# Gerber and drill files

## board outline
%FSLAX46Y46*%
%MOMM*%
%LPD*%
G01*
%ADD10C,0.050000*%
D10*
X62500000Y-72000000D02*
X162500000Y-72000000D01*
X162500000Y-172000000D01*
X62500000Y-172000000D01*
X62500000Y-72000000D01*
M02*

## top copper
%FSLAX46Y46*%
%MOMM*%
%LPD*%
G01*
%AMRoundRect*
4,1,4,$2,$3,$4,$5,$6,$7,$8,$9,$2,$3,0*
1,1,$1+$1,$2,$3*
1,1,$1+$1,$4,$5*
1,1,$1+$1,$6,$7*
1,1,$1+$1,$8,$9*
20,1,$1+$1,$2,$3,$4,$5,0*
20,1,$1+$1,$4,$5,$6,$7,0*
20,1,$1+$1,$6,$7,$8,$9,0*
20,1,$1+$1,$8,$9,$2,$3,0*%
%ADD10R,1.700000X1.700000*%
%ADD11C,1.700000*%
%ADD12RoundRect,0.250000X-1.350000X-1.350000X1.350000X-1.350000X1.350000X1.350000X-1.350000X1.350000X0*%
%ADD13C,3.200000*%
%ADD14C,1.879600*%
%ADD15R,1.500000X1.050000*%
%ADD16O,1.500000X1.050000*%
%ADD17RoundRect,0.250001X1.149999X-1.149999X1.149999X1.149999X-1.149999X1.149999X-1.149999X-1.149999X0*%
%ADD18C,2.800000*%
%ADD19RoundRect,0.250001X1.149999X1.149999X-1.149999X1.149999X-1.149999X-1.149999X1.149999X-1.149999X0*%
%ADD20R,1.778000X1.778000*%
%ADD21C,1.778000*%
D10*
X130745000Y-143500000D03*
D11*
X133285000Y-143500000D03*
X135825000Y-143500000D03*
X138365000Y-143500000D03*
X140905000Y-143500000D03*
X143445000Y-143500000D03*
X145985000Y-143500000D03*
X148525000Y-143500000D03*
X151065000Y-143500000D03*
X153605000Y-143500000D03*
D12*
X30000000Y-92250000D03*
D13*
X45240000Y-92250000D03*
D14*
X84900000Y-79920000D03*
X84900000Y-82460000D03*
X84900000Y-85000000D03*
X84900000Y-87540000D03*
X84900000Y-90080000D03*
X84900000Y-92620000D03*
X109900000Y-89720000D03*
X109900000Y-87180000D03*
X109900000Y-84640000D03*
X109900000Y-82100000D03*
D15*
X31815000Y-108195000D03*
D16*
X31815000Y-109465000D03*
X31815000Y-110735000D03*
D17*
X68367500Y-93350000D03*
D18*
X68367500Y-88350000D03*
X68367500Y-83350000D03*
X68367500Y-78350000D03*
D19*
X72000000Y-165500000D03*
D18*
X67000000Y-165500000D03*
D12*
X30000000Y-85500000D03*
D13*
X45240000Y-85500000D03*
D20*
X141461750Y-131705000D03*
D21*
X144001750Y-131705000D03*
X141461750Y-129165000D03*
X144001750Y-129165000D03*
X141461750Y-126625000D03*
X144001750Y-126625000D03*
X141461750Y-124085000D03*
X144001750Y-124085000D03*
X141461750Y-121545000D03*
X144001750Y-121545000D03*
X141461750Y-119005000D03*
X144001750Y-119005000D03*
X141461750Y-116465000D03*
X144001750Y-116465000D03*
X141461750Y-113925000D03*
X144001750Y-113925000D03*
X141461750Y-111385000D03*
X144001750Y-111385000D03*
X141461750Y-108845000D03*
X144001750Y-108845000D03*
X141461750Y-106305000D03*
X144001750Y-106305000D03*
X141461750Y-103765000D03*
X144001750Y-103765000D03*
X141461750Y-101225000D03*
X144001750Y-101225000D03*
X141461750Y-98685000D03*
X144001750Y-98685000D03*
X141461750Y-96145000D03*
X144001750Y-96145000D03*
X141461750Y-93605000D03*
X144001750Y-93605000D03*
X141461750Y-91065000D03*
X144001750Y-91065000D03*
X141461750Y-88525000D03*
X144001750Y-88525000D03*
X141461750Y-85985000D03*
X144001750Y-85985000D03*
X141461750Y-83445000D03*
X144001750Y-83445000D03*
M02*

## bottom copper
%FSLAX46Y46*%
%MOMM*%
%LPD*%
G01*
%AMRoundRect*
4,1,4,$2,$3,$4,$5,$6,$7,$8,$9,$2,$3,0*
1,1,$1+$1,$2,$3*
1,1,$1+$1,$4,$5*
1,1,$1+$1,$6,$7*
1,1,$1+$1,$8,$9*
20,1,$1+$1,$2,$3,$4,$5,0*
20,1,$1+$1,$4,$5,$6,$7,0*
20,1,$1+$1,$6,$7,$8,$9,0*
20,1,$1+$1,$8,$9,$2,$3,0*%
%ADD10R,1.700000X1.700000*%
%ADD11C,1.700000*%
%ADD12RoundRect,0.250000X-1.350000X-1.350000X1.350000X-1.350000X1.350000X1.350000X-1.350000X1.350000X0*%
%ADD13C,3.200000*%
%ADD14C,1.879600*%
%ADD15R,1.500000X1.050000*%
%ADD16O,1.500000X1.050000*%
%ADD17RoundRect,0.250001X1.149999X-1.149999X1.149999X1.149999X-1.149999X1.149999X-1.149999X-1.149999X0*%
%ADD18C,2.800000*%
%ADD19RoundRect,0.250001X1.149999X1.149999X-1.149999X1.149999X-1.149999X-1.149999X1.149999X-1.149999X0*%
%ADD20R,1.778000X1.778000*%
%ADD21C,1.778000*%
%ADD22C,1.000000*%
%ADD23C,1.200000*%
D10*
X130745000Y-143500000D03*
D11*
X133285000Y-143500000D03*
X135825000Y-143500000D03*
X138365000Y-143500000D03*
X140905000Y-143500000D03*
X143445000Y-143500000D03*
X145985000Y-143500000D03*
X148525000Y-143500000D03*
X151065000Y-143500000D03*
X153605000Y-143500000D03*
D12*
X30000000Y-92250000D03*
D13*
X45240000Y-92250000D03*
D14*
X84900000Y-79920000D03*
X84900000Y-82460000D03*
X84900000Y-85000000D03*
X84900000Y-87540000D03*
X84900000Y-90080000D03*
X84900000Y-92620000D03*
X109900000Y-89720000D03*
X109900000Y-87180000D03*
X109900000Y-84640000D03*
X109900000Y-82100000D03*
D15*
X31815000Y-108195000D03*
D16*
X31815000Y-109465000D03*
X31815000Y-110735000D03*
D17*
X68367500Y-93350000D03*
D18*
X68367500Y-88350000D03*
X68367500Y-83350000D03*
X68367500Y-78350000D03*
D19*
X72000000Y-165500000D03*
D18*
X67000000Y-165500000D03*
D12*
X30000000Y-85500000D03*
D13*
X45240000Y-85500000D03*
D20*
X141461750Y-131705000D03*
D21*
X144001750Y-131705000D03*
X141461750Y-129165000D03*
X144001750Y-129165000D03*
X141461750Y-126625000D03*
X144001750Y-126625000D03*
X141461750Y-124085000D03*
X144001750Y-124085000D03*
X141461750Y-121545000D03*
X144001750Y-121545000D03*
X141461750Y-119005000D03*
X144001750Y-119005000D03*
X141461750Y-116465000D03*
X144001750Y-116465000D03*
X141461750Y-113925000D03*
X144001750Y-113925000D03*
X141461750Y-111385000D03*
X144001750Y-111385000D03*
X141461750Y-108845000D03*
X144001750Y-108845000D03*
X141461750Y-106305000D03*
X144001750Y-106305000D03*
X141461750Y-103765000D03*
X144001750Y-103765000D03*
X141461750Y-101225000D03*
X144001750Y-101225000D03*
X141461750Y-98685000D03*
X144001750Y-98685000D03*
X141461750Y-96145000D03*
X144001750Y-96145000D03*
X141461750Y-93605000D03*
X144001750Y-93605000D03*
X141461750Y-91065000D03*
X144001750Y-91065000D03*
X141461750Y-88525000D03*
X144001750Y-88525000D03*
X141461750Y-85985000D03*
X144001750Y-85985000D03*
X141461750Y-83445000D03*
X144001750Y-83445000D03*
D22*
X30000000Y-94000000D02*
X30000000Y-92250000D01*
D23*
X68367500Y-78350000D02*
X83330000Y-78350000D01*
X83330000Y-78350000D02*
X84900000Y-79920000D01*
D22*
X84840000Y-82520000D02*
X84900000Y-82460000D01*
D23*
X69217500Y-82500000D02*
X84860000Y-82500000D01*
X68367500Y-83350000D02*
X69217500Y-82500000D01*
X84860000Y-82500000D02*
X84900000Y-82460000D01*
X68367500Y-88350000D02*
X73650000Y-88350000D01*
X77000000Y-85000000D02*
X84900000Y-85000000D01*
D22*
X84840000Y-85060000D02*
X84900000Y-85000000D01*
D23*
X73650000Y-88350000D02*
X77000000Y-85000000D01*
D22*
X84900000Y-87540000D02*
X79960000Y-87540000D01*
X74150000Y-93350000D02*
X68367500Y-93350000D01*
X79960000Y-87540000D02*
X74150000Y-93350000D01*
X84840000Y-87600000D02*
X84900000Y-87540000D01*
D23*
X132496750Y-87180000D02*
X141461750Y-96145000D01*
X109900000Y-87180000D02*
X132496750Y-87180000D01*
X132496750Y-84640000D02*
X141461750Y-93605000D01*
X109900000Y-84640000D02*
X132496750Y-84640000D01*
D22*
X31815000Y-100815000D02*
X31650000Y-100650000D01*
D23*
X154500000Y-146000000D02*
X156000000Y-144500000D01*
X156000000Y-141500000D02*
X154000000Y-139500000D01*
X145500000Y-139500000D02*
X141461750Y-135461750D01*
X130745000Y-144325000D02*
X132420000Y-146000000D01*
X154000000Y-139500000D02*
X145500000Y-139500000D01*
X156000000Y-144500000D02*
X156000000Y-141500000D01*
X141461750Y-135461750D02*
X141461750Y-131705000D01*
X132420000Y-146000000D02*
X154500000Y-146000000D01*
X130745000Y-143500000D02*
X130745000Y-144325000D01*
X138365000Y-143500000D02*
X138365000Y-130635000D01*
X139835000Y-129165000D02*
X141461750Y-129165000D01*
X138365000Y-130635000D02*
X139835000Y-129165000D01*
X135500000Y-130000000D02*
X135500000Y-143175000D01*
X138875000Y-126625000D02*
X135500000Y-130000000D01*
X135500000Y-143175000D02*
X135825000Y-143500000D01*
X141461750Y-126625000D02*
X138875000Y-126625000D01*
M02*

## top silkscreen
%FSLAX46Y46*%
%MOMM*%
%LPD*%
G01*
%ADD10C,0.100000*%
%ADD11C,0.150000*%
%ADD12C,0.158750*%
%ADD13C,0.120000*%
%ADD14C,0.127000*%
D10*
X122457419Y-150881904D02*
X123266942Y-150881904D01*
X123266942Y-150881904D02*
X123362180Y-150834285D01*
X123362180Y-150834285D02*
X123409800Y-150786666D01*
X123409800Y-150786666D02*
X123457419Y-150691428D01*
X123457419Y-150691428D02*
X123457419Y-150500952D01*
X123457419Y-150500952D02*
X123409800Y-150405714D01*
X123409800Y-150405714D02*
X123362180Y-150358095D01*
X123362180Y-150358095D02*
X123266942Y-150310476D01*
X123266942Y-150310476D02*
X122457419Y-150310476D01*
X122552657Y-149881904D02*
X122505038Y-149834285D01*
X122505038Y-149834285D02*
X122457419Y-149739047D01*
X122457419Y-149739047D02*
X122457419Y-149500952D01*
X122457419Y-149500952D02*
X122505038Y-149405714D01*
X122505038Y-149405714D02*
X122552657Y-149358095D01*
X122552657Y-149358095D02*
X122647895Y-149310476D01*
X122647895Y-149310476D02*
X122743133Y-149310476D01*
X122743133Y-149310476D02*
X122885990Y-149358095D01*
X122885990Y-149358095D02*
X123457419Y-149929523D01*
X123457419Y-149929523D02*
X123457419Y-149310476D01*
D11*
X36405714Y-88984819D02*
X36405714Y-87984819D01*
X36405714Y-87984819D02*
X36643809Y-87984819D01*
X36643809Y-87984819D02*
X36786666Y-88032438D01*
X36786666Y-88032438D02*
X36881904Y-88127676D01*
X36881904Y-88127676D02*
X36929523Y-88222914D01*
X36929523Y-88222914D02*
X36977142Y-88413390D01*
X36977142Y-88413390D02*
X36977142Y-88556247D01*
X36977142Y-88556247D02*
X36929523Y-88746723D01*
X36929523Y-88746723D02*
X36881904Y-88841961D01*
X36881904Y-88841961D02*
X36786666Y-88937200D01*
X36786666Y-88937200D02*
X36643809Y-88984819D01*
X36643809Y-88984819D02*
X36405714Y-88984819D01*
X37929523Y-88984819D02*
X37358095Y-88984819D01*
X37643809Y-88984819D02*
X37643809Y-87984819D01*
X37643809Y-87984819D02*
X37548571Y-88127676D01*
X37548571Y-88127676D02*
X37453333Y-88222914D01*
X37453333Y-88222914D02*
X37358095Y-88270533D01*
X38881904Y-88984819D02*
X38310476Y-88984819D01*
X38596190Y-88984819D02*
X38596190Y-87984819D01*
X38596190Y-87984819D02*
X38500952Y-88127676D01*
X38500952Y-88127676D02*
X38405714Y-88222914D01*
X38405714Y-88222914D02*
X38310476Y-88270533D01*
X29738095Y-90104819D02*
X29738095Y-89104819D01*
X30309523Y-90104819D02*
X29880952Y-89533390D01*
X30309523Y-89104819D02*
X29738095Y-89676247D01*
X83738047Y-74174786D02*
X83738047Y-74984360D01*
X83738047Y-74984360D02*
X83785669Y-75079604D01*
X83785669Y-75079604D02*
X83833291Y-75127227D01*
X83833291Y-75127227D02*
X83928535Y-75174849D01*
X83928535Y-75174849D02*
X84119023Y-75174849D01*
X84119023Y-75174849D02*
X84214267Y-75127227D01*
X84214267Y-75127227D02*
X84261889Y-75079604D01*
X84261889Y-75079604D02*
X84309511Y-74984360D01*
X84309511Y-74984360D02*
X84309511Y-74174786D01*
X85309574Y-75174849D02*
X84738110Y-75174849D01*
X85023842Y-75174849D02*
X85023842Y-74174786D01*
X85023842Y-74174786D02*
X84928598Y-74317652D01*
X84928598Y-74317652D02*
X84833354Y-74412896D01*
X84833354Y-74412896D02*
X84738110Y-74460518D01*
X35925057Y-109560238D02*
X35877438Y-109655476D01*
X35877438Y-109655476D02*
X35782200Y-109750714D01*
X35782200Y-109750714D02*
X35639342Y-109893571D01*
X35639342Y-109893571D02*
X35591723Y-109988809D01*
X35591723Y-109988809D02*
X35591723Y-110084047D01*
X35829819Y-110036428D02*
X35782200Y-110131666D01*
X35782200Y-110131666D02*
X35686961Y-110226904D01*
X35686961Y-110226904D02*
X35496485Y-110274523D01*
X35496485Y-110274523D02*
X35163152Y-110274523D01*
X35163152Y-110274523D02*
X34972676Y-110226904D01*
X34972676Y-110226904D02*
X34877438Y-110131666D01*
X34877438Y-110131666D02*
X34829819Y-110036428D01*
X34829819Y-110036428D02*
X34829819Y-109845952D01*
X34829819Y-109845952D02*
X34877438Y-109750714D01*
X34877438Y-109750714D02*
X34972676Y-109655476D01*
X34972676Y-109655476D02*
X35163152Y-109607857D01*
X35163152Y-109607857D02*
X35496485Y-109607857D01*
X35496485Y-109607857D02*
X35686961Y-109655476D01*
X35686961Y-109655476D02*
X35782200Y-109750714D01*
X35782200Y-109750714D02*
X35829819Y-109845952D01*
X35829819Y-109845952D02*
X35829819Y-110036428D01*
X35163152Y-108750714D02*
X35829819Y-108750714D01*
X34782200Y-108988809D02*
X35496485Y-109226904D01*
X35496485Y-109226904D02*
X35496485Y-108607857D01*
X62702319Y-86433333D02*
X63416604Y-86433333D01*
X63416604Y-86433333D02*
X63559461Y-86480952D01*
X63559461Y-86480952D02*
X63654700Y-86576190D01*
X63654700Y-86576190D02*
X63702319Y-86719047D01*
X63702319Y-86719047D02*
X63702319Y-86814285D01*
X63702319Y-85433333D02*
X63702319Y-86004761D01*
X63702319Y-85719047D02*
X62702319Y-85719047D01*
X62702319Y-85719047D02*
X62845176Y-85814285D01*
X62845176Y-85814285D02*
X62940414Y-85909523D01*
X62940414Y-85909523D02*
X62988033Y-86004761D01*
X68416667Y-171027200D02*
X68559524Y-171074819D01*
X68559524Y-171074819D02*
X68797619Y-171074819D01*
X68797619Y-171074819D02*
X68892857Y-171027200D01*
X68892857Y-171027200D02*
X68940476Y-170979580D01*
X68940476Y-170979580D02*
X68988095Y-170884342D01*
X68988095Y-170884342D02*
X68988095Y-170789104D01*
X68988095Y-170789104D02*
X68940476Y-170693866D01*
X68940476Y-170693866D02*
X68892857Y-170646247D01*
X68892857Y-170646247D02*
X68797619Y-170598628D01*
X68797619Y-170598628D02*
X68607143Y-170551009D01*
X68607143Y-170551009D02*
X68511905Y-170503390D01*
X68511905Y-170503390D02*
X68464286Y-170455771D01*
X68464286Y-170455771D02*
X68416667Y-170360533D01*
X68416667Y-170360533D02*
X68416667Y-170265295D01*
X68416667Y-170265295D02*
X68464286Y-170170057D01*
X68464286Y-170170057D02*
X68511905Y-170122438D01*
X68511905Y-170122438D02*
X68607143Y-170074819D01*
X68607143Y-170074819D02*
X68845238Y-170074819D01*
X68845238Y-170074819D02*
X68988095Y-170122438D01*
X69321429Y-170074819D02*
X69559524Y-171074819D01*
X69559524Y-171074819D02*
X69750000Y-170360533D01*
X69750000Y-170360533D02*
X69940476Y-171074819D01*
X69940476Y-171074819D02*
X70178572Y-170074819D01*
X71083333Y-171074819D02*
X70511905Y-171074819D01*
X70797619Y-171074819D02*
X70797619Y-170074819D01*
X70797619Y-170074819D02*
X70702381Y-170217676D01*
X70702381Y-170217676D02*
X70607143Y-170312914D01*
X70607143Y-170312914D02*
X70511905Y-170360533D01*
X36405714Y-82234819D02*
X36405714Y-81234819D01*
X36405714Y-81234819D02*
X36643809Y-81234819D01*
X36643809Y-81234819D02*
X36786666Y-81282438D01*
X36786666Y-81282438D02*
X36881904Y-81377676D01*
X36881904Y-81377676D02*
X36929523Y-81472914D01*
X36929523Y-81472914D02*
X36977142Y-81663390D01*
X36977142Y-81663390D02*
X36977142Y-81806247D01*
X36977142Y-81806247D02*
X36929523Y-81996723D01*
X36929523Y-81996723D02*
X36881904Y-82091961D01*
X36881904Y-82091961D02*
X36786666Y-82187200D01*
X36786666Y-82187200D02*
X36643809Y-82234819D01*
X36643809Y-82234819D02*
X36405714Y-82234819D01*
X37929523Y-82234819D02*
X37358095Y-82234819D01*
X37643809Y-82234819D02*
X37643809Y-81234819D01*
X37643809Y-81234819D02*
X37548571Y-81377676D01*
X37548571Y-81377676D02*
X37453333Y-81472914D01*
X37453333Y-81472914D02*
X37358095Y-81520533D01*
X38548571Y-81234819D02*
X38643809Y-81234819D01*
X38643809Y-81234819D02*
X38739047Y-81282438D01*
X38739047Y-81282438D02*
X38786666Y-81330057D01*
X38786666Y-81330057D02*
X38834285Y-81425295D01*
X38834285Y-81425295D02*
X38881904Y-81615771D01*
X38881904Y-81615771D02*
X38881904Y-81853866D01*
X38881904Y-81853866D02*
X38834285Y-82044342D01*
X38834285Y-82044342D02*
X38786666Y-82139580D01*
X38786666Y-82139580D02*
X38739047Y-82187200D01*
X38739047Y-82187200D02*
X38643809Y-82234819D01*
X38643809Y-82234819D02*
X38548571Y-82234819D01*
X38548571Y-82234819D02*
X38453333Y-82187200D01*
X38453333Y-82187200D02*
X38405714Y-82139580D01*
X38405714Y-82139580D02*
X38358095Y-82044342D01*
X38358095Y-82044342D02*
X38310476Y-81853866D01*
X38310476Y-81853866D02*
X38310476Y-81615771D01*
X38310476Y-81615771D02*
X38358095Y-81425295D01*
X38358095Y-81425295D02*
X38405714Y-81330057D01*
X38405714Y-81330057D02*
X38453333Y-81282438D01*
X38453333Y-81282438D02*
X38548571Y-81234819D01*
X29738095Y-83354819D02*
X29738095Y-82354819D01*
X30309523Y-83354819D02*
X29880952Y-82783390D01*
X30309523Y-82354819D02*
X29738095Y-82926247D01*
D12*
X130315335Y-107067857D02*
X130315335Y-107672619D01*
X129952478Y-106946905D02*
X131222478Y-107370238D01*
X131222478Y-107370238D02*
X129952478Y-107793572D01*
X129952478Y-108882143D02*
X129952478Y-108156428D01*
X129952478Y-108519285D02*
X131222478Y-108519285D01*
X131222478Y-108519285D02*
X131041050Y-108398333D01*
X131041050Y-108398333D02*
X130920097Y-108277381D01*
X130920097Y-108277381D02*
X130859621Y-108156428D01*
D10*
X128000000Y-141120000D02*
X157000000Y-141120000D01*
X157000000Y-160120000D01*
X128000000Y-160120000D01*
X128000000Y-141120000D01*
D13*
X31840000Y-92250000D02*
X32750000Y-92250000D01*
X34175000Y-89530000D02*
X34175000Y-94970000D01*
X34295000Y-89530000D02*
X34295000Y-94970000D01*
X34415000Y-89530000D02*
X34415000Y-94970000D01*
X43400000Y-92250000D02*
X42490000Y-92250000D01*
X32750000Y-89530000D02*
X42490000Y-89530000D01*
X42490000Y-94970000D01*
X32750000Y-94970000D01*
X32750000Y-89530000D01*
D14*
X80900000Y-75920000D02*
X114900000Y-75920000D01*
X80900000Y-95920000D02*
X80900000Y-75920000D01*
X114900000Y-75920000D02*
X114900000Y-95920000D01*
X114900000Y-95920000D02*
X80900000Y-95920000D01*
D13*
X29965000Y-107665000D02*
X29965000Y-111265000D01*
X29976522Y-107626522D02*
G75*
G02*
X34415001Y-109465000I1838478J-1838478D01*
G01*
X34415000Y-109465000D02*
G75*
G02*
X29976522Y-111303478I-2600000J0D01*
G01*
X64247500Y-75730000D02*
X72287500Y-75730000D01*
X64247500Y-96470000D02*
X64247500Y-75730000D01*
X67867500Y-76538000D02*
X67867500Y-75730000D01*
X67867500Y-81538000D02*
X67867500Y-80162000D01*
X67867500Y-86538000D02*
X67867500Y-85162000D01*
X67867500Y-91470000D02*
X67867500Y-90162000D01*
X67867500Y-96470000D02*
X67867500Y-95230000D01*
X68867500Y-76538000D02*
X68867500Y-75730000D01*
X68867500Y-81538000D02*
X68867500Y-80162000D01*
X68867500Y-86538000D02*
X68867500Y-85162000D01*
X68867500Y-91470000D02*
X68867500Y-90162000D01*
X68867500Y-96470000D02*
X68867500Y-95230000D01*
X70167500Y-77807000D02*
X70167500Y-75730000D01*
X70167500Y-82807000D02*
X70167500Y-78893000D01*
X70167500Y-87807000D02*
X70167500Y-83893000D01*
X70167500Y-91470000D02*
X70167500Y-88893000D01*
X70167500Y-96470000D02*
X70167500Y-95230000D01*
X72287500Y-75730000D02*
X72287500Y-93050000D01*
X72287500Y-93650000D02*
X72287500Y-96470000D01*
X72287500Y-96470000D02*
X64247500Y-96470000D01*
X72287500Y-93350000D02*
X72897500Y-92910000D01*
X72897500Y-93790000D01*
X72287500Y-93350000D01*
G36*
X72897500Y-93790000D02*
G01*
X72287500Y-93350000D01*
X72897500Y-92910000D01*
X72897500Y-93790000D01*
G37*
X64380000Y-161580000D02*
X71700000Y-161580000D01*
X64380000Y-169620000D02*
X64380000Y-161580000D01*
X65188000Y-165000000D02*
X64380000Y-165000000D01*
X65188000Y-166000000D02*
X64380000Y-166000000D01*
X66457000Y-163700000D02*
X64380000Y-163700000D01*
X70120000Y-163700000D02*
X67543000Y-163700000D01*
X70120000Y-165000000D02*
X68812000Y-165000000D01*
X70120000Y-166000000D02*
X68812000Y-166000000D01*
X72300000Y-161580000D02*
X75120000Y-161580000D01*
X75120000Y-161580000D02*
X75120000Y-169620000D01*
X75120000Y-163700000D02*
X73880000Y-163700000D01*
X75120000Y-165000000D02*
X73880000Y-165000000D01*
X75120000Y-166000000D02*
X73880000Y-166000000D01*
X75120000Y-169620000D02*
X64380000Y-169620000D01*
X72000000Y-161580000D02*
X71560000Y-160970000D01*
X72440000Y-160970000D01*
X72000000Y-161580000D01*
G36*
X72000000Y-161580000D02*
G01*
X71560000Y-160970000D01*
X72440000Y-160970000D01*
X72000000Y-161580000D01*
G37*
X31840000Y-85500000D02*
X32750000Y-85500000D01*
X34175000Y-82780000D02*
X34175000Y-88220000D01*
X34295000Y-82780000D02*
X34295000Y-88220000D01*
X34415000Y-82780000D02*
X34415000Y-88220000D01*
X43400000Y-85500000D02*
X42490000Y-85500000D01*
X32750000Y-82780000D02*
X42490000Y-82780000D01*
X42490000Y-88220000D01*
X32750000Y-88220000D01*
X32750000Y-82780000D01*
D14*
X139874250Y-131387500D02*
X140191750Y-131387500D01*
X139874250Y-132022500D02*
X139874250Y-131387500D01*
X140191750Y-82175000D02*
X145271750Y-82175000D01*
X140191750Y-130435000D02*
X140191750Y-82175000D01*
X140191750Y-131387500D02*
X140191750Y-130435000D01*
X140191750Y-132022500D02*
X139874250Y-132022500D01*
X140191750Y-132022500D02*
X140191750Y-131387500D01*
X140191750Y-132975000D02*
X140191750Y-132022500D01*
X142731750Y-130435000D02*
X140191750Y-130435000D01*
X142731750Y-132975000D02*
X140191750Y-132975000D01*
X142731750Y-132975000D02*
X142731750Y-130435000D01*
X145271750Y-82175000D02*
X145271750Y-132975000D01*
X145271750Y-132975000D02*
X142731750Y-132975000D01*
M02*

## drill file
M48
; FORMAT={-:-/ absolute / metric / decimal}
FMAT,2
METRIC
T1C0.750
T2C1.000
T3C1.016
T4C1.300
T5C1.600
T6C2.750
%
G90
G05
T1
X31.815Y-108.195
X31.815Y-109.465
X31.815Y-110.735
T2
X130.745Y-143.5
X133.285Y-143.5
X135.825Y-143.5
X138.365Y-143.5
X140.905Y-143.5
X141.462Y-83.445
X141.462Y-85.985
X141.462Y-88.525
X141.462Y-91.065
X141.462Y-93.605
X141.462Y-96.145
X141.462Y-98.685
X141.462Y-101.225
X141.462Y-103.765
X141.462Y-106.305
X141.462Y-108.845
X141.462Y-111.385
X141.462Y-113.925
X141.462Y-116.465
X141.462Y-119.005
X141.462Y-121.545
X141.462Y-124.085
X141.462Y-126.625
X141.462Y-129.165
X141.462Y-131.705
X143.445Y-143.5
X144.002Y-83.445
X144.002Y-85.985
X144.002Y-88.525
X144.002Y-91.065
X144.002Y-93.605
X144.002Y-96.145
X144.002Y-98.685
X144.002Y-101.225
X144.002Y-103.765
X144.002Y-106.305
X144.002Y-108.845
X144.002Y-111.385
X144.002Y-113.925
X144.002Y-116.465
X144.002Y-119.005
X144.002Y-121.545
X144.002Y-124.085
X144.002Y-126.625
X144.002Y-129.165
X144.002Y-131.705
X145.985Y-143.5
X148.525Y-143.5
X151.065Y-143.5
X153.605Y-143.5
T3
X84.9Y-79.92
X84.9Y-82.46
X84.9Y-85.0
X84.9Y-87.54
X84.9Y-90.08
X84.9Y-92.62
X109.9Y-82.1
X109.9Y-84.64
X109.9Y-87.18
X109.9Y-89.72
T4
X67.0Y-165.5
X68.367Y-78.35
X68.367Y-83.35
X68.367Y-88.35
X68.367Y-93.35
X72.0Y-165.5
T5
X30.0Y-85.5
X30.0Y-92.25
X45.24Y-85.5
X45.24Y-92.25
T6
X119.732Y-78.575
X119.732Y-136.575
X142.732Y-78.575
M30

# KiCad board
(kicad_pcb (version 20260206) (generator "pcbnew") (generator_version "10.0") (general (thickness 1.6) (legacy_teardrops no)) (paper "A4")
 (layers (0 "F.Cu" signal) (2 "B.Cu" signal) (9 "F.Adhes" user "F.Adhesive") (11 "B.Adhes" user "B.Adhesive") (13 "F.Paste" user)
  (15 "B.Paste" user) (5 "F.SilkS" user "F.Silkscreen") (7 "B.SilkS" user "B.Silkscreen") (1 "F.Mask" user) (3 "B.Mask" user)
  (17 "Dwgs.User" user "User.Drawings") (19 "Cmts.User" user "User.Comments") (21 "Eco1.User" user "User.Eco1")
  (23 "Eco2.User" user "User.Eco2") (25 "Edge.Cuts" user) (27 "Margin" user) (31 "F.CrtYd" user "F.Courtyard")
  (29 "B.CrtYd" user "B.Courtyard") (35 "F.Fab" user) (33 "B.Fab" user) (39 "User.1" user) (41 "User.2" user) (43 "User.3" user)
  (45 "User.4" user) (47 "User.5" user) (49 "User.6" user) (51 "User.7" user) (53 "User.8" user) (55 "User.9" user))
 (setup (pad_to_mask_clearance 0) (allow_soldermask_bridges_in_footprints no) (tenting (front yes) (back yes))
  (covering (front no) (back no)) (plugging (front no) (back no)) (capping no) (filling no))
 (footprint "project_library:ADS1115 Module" (layer "F.Cu") (at 123.5 150.12 90)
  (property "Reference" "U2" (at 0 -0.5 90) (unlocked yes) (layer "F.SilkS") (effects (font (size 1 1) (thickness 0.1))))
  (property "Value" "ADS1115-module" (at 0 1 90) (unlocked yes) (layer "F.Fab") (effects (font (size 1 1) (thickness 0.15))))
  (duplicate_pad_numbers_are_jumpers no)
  (fp_rect (start -10 4.5) (end 9 33.5) (stroke (width 0.1) (type default)) (fill no) (layer "F.SilkS"))
  (pad "1" thru_hole rect (at 6.62 7.245 90) (size 1.7 1.7) (drill 1) (layers "*.Cu" "*.Mask") (remove_unused_layers no) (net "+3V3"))
  (pad "2" thru_hole circle (at 6.62 9.785 90) (size 1.7 1.7) (drill 1) (layers "*.Cu" "*.Mask") (remove_unused_layers no))
  (pad "3" thru_hole circle (at 6.62 12.325 90) (size 1.7 1.7) (drill 1) (layers "*.Cu" "*.Mask") (remove_unused_layers no) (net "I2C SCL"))
  (pad "4" thru_hole circle (at 6.62 14.865 90) (size 1.7 1.7) (drill 1) (layers "*.Cu" "*.Mask") (remove_unused_layers no) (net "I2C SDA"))
  (pad "5" thru_hole circle (at 6.62 17.405 90) (size 1.7 1.7) (drill 1) (layers "*.Cu" "*.Mask") (remove_unused_layers no)
   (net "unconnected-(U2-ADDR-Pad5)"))
  (pad "6" thru_hole circle (at 6.62 19.945 90) (size 1.7 1.7) (drill 1) (layers "*.Cu" "*.Mask") (remove_unused_layers no)
   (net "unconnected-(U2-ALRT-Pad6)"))
  (pad "7" thru_hole circle (at 6.62 22.485 90) (size 1.7 1.7) (drill 1) (layers "*.Cu" "*.Mask") (remove_unused_layers no)
   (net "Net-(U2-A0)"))
  (pad "8" thru_hole circle (at 6.62 25.025 90) (size 1.7 1.7) (drill 1) (layers "*.Cu" "*.Mask") (remove_unused_layers no)
   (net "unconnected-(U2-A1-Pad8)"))
  (pad "9" thru_hole circle (at 6.62 27.565 90) (size 1.7 1.7) (drill 1) (layers "*.Cu" "*.Mask") (remove_unused_layers no)
   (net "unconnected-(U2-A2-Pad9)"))
  (pad "10" thru_hole circle (at 6.62 30.105 90) (size 1.7 1.7) (drill 1) (layers "*.Cu" "*.Mask") (remove_unused_layers no)
   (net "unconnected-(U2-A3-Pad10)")))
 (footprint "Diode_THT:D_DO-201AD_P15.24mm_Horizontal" (layer "F.Cu") (at 30 92.25)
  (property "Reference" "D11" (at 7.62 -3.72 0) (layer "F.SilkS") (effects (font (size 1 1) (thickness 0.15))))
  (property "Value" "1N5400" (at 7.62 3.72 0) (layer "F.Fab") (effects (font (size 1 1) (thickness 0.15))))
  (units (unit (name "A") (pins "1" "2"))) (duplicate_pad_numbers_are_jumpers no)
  (fp_line (start 1.84 0) (end 2.75 0) (stroke (width 0.12) (type solid)) (layer "F.SilkS"))
  (fp_line (start 4.175 -2.72) (end 4.175 2.72) (stroke (width 0.12) (type solid)) (layer "F.SilkS"))
  (fp_line (start 4.295 -2.72) (end 4.295 2.72) (stroke (width 0.12) (type solid)) (layer "F.SilkS"))
  (fp_line (start 4.415 -2.72) (end 4.415 2.72) (stroke (width 0.12) (type solid)) (layer "F.SilkS"))
  (fp_line (start 13.4 0) (end 12.49 0) (stroke (width 0.12) (type solid)) (layer "F.SilkS"))
  (fp_rect (start 2.75 -2.72) (end 12.49 2.72) (stroke (width 0.12) (type solid)) (fill no) (layer "F.SilkS"))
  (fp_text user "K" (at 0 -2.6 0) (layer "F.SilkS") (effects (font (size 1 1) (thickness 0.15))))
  (pad "1" thru_hole roundrect (at 0 0) (size 3.2 3.2) (drill 1.6) (layers "*.Cu" "*.Mask") (remove_unused_layers no)
   (roundrect_rratio 0.078125) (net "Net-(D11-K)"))
  (pad "2" thru_hole circle (at 15.24 0) (size 3.2 3.2) (drill 1.6) (layers "*.Cu" "*.Mask") (remove_unused_layers no) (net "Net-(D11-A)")))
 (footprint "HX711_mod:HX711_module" (layer "F.Cu") (at 97.9 85.92)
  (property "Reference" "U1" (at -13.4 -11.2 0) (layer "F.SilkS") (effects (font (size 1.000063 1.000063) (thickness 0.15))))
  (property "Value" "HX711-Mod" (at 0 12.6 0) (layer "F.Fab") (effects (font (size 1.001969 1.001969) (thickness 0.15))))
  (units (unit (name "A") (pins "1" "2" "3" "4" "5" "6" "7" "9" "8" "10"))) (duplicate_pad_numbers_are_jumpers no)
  (fp_line (start -17 -10) (end 17 -10) (stroke (width 0.127) (type solid)) (layer "F.SilkS"))
  (fp_line (start -17 10) (end -17 -10) (stroke (width 0.127) (type solid)) (layer "F.SilkS"))
  (fp_line (start 17 -10) (end 17 10) (stroke (width 0.127) (type solid)) (layer "F.SilkS"))
  (fp_line (start 17 10) (end -17 10) (stroke (width 0.127) (type solid)) (layer "F.SilkS"))
  (pad "1" thru_hole circle (at -13 -6) (size 1.8796 1.8796) (drill 1.016) (layers "*.Cu" "*.Mask") (remove_unused_layers no)
   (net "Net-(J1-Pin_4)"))
  (pad "2" thru_hole circle (at -13 -3.46) (size 1.8796 1.8796) (drill 1.016) (layers "*.Cu" "*.Mask") (remove_unused_layers no)
   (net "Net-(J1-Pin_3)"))
  (pad "3" thru_hole circle (at -13 -0.92) (size 1.8796 1.8796) (drill 1.016) (layers "*.Cu" "*.Mask") (remove_unused_layers no)
   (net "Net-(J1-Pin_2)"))
  (pad "4" thru_hole circle (at -13 1.62) (size 1.8796 1.8796) (drill 1.016) (layers "*.Cu" "*.Mask") (remove_unused_layers no)
   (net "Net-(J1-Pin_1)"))
  (pad "5" thru_hole circle (at -13 4.16) (size 1.8796 1.8796) (drill 1.016) (layers "*.Cu" "*.Mask") (remove_unused_layers no)
   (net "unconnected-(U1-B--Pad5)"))
  (pad "6" thru_hole circle (at -13 6.7) (size 1.8796 1.8796) (drill 1.016) (layers "*.Cu" "*.Mask") (remove_unused_layers no)
   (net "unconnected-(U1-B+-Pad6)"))
  (pad "7" thru_hole circle (at 12 3.8) (size 1.8796 1.8796) (drill 1.016) (layers "*.Cu" "*.Mask") (remove_unused_layers no)
   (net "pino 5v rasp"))
  (pad "8" thru_hole circle (at 12 1.26) (size 1.8796 1.8796) (drill 1.016) (layers "*.Cu" "*.Mask") (remove_unused_layers no)
   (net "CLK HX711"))
  (pad "9" thru_hole circle (at 12 -1.28) (size 1.8796 1.8796) (drill 1.016) (layers "*.Cu" "*.Mask") (remove_unused_layers no)
   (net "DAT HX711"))
  (pad "10" thru_hole circle (at 12 -3.82) (size 1.8796 1.8796) (drill 1.016) (layers "*.Cu" "*.Mask") (remove_unused_layers no)
   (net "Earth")))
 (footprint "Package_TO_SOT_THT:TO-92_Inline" (layer "F.Cu") (at 31.815 108.195 -90)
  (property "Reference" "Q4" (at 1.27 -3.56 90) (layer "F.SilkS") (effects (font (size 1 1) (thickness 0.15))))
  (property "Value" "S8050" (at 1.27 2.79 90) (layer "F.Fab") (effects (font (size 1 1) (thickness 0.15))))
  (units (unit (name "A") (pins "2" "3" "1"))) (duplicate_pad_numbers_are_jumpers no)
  (fp_line (start -0.53 1.85) (end 3.07 1.85) (stroke (width 0.12) (type solid)) (layer "F.SilkS"))
  (fp_arc (start -0.568478 1.838478) (mid -1.132087 -0.994977) (end 1.27 -2.6) (stroke (width 0.12) (type solid)) (layer "F.SilkS"))
  (fp_arc (start 1.27 -2.6) (mid 3.672087 -0.994977) (end 3.108478 1.838478) (stroke (width 0.12) (type solid)) (layer "F.SilkS"))
  (pad "1" thru_hole rect (at 0 0 270) (size 1.05 1.5) (drill 0.75) (layers "*.Cu" "*.Mask") (remove_unused_layers no) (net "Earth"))
  (pad "2" thru_hole oval (at 1.27 0 270) (size 1.05 1.5) (drill 0.75) (layers "*.Cu" "*.Mask") (remove_unused_layers no) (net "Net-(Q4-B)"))
  (pad "3" thru_hole oval (at 2.54 0 270) (size 1.05 1.5) (drill 0.75) (layers "*.Cu" "*.Mask") (remove_unused_layers no)
   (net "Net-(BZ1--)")))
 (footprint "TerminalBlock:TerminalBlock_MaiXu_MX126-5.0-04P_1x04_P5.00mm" (layer "F.Cu") (at 68.3675 93.35 90)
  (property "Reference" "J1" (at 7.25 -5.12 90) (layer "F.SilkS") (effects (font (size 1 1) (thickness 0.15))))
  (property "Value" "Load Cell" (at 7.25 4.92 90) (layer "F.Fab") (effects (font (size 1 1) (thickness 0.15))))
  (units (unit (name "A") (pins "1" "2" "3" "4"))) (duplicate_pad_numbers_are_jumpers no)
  (fp_line (start 17.62 -4.12) (end 17.62 3.92) (stroke (width 0.12) (type solid)) (layer "F.SilkS"))
  (fp_line (start -3.12 -4.12) (end 17.62 -4.12) (stroke (width 0.12) (type solid)) (layer "F.SilkS"))
  (fp_line (start 16.812 -0.5) (end 17.62 -0.5) (stroke (width 0.12) (type solid)) (layer "F.SilkS"))
  (fp_line (start 11.812 -0.5) (end 13.188 -0.5) (stroke (width 0.12) (type solid)) (layer "F.SilkS"))
  (fp_line (start 6.812 -0.5) (end 8.188 -0.5) (stroke (width 0.12) (type solid)) (layer "F.SilkS"))
  (fp_line (start 1.88 -0.5) (end 3.188 -0.5) (stroke (width 0.12) (type solid)) (layer "F.SilkS"))
  (fp_line (start -3.12 -0.5) (end -1.88 -0.5) (stroke (width 0.12) (type solid)) (layer "F.SilkS"))
  (fp_line (start 16.812 0.5) (end 17.62 0.5) (stroke (width 0.12) (type solid)) (layer "F.SilkS"))
  (fp_line (start 11.812 0.5) (end 13.188 0.5) (stroke (width 0.12) (type solid)) (layer "F.SilkS"))
  (fp_line (start 6.812 0.5) (end 8.188 0.5) (stroke (width 0.12) (type solid)) (layer "F.SilkS"))
  (fp_line (start 1.88 0.5) (end 3.188 0.5) (stroke (width 0.12) (type solid)) (layer "F.SilkS"))
  (fp_line (start -3.12 0.5) (end -1.88 0.5) (stroke (width 0.12) (type solid)) (layer "F.SilkS"))
  (fp_line (start 15.543 1.8) (end 17.62 1.8) (stroke (width 0.12) (type solid)) (layer "F.SilkS"))
  (fp_line (start 10.543 1.8) (end 14.457 1.8) (stroke (width 0.12) (type solid)) (layer "F.SilkS"))
  (fp_line (start 5.543 1.8) (end 9.457 1.8) (stroke (width 0.12) (type solid)) (layer "F.SilkS"))
  (fp_line (start 1.88 1.8) (end 4.457 1.8) (stroke (width 0.12) (type solid)) (layer "F.SilkS"))
  (fp_line (start -3.12 1.8) (end -1.88 1.8) (stroke (width 0.12) (type solid)) (layer "F.SilkS"))
  (fp_line (start 17.62 3.92) (end 0.3 3.92) (stroke (width 0.12) (type solid)) (layer "F.SilkS"))
  (fp_line (start -0.3 3.92) (end -3.12 3.92) (stroke (width 0.12) (type solid)) (layer "F.SilkS"))
  (fp_line (start -3.12 3.92) (end -3.12 -4.12) (stroke (width 0.12) (type solid)) (layer "F.SilkS"))
  (fp_poly (pts (xy 0 3.92) (xy 0.44 4.53) (xy -0.44 4.53)) (stroke (width 0.12) (type solid)) (fill yes) (layer "F.SilkS"))
  (pad "1" thru_hole roundrect (at 0 0 90) (size 2.8 2.8) (drill 1.3) (layers "*.Cu" "*.Mask") (remove_unused_layers no)
   (roundrect_rratio 0.089286) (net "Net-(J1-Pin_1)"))
  (pad "2" thru_hole circle (at 5 0 90) (size 2.8 2.8) (drill 1.3) (layers "*.Cu" "*.Mask") (remove_unused_layers no) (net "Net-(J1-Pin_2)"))
  (pad "3" thru_hole circle (at 10 0 90) (size 2.8 2.8) (drill 1.3) (layers "*.Cu" "*.Mask") (remove_unused_layers no)
   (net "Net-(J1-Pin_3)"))
  (pad "4" thru_hole circle (at 15 0 90) (size 2.8 2.8) (drill 1.3) (layers "*.Cu" "*.Mask") (remove_unused_layers no)
   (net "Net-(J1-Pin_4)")))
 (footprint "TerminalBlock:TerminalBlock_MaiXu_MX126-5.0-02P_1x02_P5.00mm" (layer "F.Cu") (at 72 165.5 180)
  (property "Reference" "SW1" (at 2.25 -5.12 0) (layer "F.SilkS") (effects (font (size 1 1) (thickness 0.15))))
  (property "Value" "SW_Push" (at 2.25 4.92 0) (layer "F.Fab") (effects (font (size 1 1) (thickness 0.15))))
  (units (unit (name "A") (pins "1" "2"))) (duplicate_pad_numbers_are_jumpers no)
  (fp_line (start 7.62 3.92) (end 0.3 3.92) (stroke (width 0.12) (type solid)) (layer "F.SilkS"))
  (fp_line (start 7.62 -4.12) (end 7.62 3.92) (stroke (width 0.12) (type solid)) (layer "F.SilkS"))
  (fp_line (start 6.812 0.5) (end 7.62 0.5) (stroke (width 0.12) (type solid)) (layer "F.SilkS"))
  (fp_line (start 6.812 -0.5) (end 7.62 -0.5) (stroke (width 0.12) (type solid)) (layer "F.SilkS"))
  (fp_line (start 5.543 1.8) (end 7.62 1.8) (stroke (width 0.12) (type solid)) (layer "F.SilkS"))
  (fp_line (start 1.88 1.8) (end 4.457 1.8) (stroke (width 0.12) (type solid)) (layer "F.SilkS"))
  (fp_line (start 1.88 0.5) (end 3.188 0.5) (stroke (width 0.12) (type solid)) (layer "F.SilkS"))
  (fp_line (start 1.88 -0.5) (end 3.188 -0.5) (stroke (width 0.12) (type solid)) (layer "F.SilkS"))
  (fp_line (start -0.3 3.92) (end -3.12 3.92) (stroke (width 0.12) (type solid)) (layer "F.SilkS"))
  (fp_line (start -3.12 3.92) (end -3.12 -4.12) (stroke (width 0.12) (type solid)) (layer "F.SilkS"))
  (fp_line (start -3.12 1.8) (end -1.88 1.8) (stroke (width 0.12) (type solid)) (layer "F.SilkS"))
  (fp_line (start -3.12 0.5) (end -1.88 0.5) (stroke (width 0.12) (type solid)) (layer "F.SilkS"))
  (fp_line (start -3.12 -0.5) (end -1.88 -0.5) (stroke (width 0.12) (type solid)) (layer "F.SilkS"))
  (fp_line (start -3.12 -4.12) (end 7.62 -4.12) (stroke (width 0.12) (type solid)) (layer "F.SilkS"))
  (fp_poly (pts (xy 0 3.92) (xy 0.44 4.53) (xy -0.44 4.53)) (stroke (width 0.12) (type solid)) (fill yes) (layer "F.SilkS"))
  (pad "1" thru_hole roundrect (at 0 0 180) (size 2.8 2.8) (drill 1.3) (layers "*.Cu" "*.Mask") (remove_unused_layers no)
   (roundrect_rratio 0.089286) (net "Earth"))
  (pad "2" thru_hole circle (at 5 0 180) (size 2.8 2.8) (drill 1.3) (layers "*.Cu" "*.Mask") (remove_unused_layers no) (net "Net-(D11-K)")))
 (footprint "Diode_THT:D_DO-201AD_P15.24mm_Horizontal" (layer "F.Cu") (at 30 85.5)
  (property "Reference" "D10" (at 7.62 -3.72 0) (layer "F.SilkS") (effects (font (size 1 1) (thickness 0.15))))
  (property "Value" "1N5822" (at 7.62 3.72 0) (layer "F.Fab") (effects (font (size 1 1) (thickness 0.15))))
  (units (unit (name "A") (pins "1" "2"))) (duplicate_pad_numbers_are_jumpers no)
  (fp_line (start 1.84 0) (end 2.75 0) (stroke (width 0.12) (type solid)) (layer "F.SilkS"))
  (fp_line (start 4.175 -2.72) (end 4.175 2.72) (stroke (width 0.12) (type solid)) (layer "F.SilkS"))
  (fp_line (start 4.295 -2.72) (end 4.295 2.72) (stroke (width 0.12) (type solid)) (layer "F.SilkS"))
  (fp_line (start 4.415 -2.72) (end 4.415 2.72) (stroke (width 0.12) (type solid)) (layer "F.SilkS"))
  (fp_line (start 13.4 0) (end 12.49 0) (stroke (width 0.12) (type solid)) (layer "F.SilkS"))
  (fp_rect (start 2.75 -2.72) (end 12.49 2.72) (stroke (width 0.12) (type solid)) (fill no) (layer "F.SilkS"))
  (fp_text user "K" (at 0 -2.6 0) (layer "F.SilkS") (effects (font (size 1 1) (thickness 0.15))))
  (pad "1" thru_hole roundrect (at 0 0) (size 3.2 3.2) (drill 1.6) (layers "*.Cu" "*.Mask") (remove_unused_layers no)
   (roundrect_rratio 0.078125) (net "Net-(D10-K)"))
  (pad "2" thru_hole circle (at 15.24 0) (size 3.2 3.2) (drill 1.6) (layers "*.Cu" "*.Mask") (remove_unused_layers no) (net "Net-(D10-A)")))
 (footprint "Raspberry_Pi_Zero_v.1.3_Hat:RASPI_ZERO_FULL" (layer "F.Cu") (at 116.23175 75.075 -90)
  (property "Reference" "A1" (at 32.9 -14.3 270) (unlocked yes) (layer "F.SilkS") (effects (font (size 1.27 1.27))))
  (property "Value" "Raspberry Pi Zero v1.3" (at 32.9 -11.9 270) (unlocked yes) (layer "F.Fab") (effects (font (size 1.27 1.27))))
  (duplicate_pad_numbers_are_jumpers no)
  (fp_line (start 56.3125 -23.6425) (end 56.3125 -23.96) (stroke (width 0.127) (type solid)) (layer "F.SilkS"))
  (fp_line (start 56.9475 -23.6425) (end 56.3125 -23.6425) (stroke (width 0.127) (type solid)) (layer "F.SilkS"))
  (fp_line (start 7.1 -23.96) (end 7.1 -29.04) (stroke (width 0.127) (type solid)) (layer "F.SilkS"))
  (fp_line (start 55.36 -23.96) (end 7.1 -23.96) (stroke (width 0.127) (type solid)) (layer "F.SilkS"))
  (fp_line (start 56.3125 -23.96) (end 55.36 -23.96) (stroke (width 0.127) (type solid)) (layer "F.SilkS"))
  (fp_line (start 56.9475 -23.96) (end 56.9475 -23.6425) (stroke (width 0.127) (type solid)) (layer "F.SilkS"))
  (fp_line (start 56.9475 -23.96) (end 56.3125 -23.96) (stroke (width 0.127) (type solid)) (layer "F.SilkS"))
  (fp_line (start 57.9 -23.96) (end 56.9475 -23.96) (stroke (width 0.127) (type solid)) (layer "F.SilkS"))
  (fp_line (start 55.36 -26.5) (end 55.36 -23.96) (stroke (width 0.127) (type solid)) (layer "F.SilkS"))
  (fp_line (start 57.9 -26.5) (end 57.9 -23.96) (stroke (width 0.127) (type solid)) (layer "F.SilkS"))
  (fp_line (start 57.9 -26.5) (end 55.36 -26.5) (stroke (width 0.127) (type solid)) (layer "F.SilkS"))
  (fp_line (start 7.1 -29.04) (end 57.9 -29.04) (stroke (width 0.127) (type solid)) (layer "F.SilkS"))
  (fp_line (start 57.9 -29.04) (end 57.9 -26.5) (stroke (width 0.127) (type solid)) (layer "F.SilkS"))
  (pad "" np_thru_hole circle (at 3.5 -26.5 270) (size 2.75 2.75) (drill 2.75) (layers "*.Cu" "*.Mask"))
  (pad "" np_thru_hole circle (at 3.5 -3.5 270) (size 2.75 2.75) (drill 2.75) (layers "*.Cu" "*.Mask"))
  (pad "" np_thru_hole circle (at 61.5 -3.5 270) (size 2.75 2.75) (drill 2.75) (layers "*.Cu" "*.Mask"))
  (pad "1" thru_hole rect (at 56.63 -25.23 270) (size 1.778 1.778) (drill 1) (layers "*.Cu" "*.Mask") (remove_unused_layers no) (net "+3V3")
   (solder_mask_margin 0.1016) (thermal_bridge_angle 0))
  (pad "2" thru_hole circle (at 56.63 -27.77 270) (size 1.778 1.778) (drill 1) (layers "*.Cu" "*.Mask") (remove_unused_layers no)
   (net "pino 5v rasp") (solder_mask_margin 0.1016) (thermal_bridge_angle 0))
  (pad "3" thru_hole circle (at 54.09 -25.23 270) (size 1.778 1.778) (drill 1) (layers "*.Cu" "*.Mask") (remove_unused_layers no)
   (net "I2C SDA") (solder_mask_margin 0.1016) (thermal_bridge_angle 0))
  (pad "4" thru_hole circle (at 54.09 -27.77 270) (size 1.778 1.778) (drill 1) (layers "*.Cu" "*.Mask") (remove_unused_layers no)
   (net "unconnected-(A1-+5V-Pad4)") (solder_mask_margin 0.1016) (thermal_bridge_angle 0))
  (pad "5" thru_hole circle (at 51.55 -25.23 270) (size 1.778 1.778) (drill 1) (layers "*.Cu" "*.Mask") (remove_unused_layers no)
   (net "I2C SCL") (solder_mask_margin 0.1016) (thermal_bridge_angle 0))
  (pad "6" thru_hole circle (at 51.55 -27.77 270) (size 1.778 1.778) (drill 1) (layers "*.Cu" "*.Mask") (remove_unused_layers no)
   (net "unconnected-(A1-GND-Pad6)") (solder_mask_margin 0.1016) (thermal_bridge_angle 0))
  (pad "7" thru_hole circle (at 49.01 -25.23 270) (size 1.778 1.778) (drill 1) (layers "*.Cu" "*.Mask") (remove_unused_layers no)
   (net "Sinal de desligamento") (solder_mask_margin 0.1016) (thermal_bridge_angle 0))
  (pad "8" thru_hole circle (at 49.01 -27.77 270) (size 1.778 1.778) (drill 1) (layers "*.Cu" "*.Mask") (remove_unused_layers no)
   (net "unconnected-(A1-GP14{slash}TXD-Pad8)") (solder_mask_margin 0.1016) (thermal_bridge_angle 0))
  (pad "9" thru_hole circle (at 46.47 -25.23 270) (size 1.778 1.778) (drill 1) (layers "*.Cu" "*.Mask") (remove_unused_layers no)
   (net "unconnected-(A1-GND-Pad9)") (solder_mask_margin 0.1016) (thermal_bridge_angle 0))
  (pad "10" thru_hole circle (at 46.47 -27.77 270) (size 1.778 1.778) (drill 1) (layers "*.Cu" "*.Mask") (remove_unused_layers no)
   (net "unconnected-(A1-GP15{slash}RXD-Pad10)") (solder_mask_margin 0.1016) (thermal_bridge_angle 0))
  (pad "11" thru_hole circle (at 43.93 -25.23 270) (size 1.778 1.778) (drill 1) (layers "*.Cu" "*.Mask") (remove_unused_layers no)
   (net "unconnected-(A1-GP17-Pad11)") (solder_mask_margin 0.1016) (thermal_bridge_angle 0))
  (pad "12" thru_hole circle (at 43.93 -27.77 270) (size 1.778 1.778) (drill 1) (layers "*.Cu" "*.Mask") (remove_unused_layers no)
   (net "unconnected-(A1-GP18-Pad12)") (solder_mask_margin 0.1016) (thermal_bridge_angle 0))
  (pad "13" thru_hole circle (at 41.39 -25.23 270) (size 1.778 1.778) (drill 1) (layers "*.Cu" "*.Mask") (remove_unused_layers no)
   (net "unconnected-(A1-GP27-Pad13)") (solder_mask_margin 0.1016) (thermal_bridge_angle 0))
  (pad "14" thru_hole circle (at 41.39 -27.77 270) (size 1.778 1.778) (drill 1) (layers "*.Cu" "*.Mask") (remove_unused_layers no)
   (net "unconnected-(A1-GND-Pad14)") (solder_mask_margin 0.1016) (thermal_bridge_angle 0))
  (pad "15" thru_hole circle (at 38.85 -25.23 270) (size 1.778 1.778) (drill 1) (layers "*.Cu" "*.Mask") (remove_unused_layers no)
   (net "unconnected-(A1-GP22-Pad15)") (solder_mask_margin 0.1016) (thermal_bridge_angle 0))
  (pad "16" thru_hole circle (at 38.85 -27.77 270) (size 1.778 1.778) (drill 1) (layers "*.Cu" "*.Mask") (remove_unused_layers no)
   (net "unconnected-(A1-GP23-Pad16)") (solder_mask_margin 0.1016) (thermal_bridge_angle 0))
  (pad "17" thru_hole circle (at 36.31 -25.23 270) (size 1.778 1.778) (drill 1) (layers "*.Cu" "*.Mask") (remove_unused_layers no)
   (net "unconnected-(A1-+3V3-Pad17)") (solder_mask_margin 0.1016) (thermal_bridge_angle 0))
  (pad "18" thru_hole circle (at 36.31 -27.77 270) (size 1.778 1.778) (drill 1) (layers "*.Cu" "*.Mask") (remove_unused_layers no)
   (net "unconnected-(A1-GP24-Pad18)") (solder_mask_margin 0.1016) (thermal_bridge_angle 0))
  (pad "19" thru_hole circle (at 33.77 -25.23 270) (size 1.778 1.778) (drill 1) (layers "*.Cu" "*.Mask") (remove_unused_layers no)
   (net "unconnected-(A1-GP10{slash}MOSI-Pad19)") (solder_mask_margin 0.1016) (thermal_bridge_angle 0))
  (pad "20" thru_hole circle (at 33.77 -27.77 270) (size 1.778 1.778) (drill 1) (layers "*.Cu" "*.Mask") (remove_unused_layers no)
   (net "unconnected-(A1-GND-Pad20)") (solder_mask_margin 0.1016) (thermal_bridge_angle 0))
  (pad "21" thru_hole circle (at 31.23 -25.23 270) (size 1.778 1.778) (drill 1) (layers "*.Cu" "*.Mask") (remove_unused_layers no)
   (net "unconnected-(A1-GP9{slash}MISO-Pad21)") (solder_mask_margin 0.1016) (thermal_bridge_angle 0))
  (pad "22" thru_hole circle (at 31.23 -27.77 270) (size 1.778 1.778) (drill 1) (layers "*.Cu" "*.Mask") (remove_unused_layers no)
   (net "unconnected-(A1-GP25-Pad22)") (solder_mask_margin 0.1016) (thermal_bridge_angle 0))
  (pad "23" thru_hole circle (at 28.69 -25.23 270) (size 1.778 1.778) (drill 1) (layers "*.Cu" "*.Mask") (remove_unused_layers no)
   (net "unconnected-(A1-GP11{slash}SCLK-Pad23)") (solder_mask_margin 0.1016) (thermal_bridge_angle 0))
  (pad "24" thru_hole circle (at 28.69 -27.77 270) (size 1.778 1.778) (drill 1) (layers "*.Cu" "*.Mask") (remove_unused_layers no)
   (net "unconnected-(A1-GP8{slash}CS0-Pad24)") (solder_mask_margin 0.1016) (thermal_bridge_angle 0))
  (pad "25" thru_hole circle (at 26.15 -25.23 270) (size 1.778 1.778) (drill 1) (layers "*.Cu" "*.Mask") (remove_unused_layers no)
   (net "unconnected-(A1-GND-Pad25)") (solder_mask_margin 0.1016) (thermal_bridge_angle 0))
  (pad "26" thru_hole circle (at 26.15 -27.77 270) (size 1.778 1.778) (drill 1) (layers "*.Cu" "*.Mask") (remove_unused_layers no)
   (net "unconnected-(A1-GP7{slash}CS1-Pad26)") (solder_mask_margin 0.1016) (thermal_bridge_angle 0))
  (pad "27" thru_hole circle (at 23.61 -25.23 270) (size 1.778 1.778) (drill 1) (layers "*.Cu" "*.Mask") (remove_unused_layers no)
   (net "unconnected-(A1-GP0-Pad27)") (solder_mask_margin 0.1016) (thermal_bridge_angle 0))
  (pad "28" thru_hole circle (at 23.61 -27.77 270) (size 1.778 1.778) (drill 1) (layers "*.Cu" "*.Mask") (remove_unused_layers no)
   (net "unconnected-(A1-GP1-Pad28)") (solder_mask_margin 0.1016) (thermal_bridge_angle 0))
  (pad "29" thru_hole circle (at 21.07 -25.23 270) (size 1.778 1.778) (drill 1) (layers "*.Cu" "*.Mask") (remove_unused_layers no)
   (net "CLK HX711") (solder_mask_margin 0.1016) (thermal_bridge_angle 0))
  (pad "30" thru_hole circle (at 21.07 -27.77 270) (size 1.778 1.778) (drill 1) (layers "*.Cu" "*.Mask") (remove_unused_layers no)
   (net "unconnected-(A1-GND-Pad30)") (solder_mask_margin 0.1016) (thermal_bridge_angle 0))
  (pad "31" thru_hole circle (at 18.53 -25.23 270) (size 1.778 1.778) (drill 1) (layers "*.Cu" "*.Mask") (remove_unused_layers no)
   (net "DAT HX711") (solder_mask_margin 0.1016) (thermal_bridge_angle 0))
  (pad "32" thru_hole circle (at 18.53 -27.77 270) (size 1.778 1.778) (drill 1) (layers "*.Cu" "*.Mask") (remove_unused_layers no)
   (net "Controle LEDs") (solder_mask_margin 0.1016) (thermal_bridge_angle 0))
  (pad "33" thru_hole circle (at 15.99 -25.23 270) (size 1.778 1.778) (drill 1) (layers "*.Cu" "*.Mask") (remove_unused_layers no)
   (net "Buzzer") (solder_mask_margin 0.1016) (thermal_bridge_angle 0))
  (pad "34" thru_hole circle (at 15.99 -27.77 270) (size 1.778 1.778) (drill 1) (layers "*.Cu" "*.Mask") (remove_unused_layers no)
   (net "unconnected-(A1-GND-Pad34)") (solder_mask_margin 0.1016) (thermal_bridge_angle 0))
  (pad "35" thru_hole circle (at 13.45 -25.23 270) (size 1.778 1.778) (drill 1) (layers "*.Cu" "*.Mask") (remove_unused_layers no)
   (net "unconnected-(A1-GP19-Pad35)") (solder_mask_margin 0.1016) (thermal_bridge_angle 0))
  (pad "36" thru_hole circle (at 13.45 -27.77 270) (size 1.778 1.778) (drill 1) (layers "*.Cu" "*.Mask") (remove_unused_layers no)
   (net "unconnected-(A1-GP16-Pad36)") (solder_mask_margin 0.1016) (thermal_bridge_angle 0))
  (pad "37" thru_hole circle (at 10.91 -25.23 270) (size 1.778 1.778) (drill 1) (layers "*.Cu" "*.Mask") (remove_unused_layers no)
   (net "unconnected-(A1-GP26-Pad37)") (solder_mask_margin 0.1016) (thermal_bridge_angle 0))
  (pad "38" thru_hole circle (at 10.91 -27.77 270) (size 1.778 1.778) (drill 1) (layers "*.Cu" "*.Mask") (remove_unused_layers no)
   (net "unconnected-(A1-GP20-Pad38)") (solder_mask_margin 0.1016) (thermal_bridge_angle 0))
  (pad "39" thru_hole circle (at 8.37 -25.23 270) (size 1.778 1.778) (drill 1) (layers "*.Cu" "*.Mask") (remove_unused_layers no)
   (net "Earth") (solder_mask_margin 0.1016) (thermal_bridge_angle 0))
  (pad "40" thru_hole circle (at 8.37 -27.77 270) (size 1.778 1.778) (drill 1) (layers "*.Cu" "*.Mask") (remove_unused_layers no)
   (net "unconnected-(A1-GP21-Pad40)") (solder_mask_margin 0.1016) (thermal_bridge_angle 0))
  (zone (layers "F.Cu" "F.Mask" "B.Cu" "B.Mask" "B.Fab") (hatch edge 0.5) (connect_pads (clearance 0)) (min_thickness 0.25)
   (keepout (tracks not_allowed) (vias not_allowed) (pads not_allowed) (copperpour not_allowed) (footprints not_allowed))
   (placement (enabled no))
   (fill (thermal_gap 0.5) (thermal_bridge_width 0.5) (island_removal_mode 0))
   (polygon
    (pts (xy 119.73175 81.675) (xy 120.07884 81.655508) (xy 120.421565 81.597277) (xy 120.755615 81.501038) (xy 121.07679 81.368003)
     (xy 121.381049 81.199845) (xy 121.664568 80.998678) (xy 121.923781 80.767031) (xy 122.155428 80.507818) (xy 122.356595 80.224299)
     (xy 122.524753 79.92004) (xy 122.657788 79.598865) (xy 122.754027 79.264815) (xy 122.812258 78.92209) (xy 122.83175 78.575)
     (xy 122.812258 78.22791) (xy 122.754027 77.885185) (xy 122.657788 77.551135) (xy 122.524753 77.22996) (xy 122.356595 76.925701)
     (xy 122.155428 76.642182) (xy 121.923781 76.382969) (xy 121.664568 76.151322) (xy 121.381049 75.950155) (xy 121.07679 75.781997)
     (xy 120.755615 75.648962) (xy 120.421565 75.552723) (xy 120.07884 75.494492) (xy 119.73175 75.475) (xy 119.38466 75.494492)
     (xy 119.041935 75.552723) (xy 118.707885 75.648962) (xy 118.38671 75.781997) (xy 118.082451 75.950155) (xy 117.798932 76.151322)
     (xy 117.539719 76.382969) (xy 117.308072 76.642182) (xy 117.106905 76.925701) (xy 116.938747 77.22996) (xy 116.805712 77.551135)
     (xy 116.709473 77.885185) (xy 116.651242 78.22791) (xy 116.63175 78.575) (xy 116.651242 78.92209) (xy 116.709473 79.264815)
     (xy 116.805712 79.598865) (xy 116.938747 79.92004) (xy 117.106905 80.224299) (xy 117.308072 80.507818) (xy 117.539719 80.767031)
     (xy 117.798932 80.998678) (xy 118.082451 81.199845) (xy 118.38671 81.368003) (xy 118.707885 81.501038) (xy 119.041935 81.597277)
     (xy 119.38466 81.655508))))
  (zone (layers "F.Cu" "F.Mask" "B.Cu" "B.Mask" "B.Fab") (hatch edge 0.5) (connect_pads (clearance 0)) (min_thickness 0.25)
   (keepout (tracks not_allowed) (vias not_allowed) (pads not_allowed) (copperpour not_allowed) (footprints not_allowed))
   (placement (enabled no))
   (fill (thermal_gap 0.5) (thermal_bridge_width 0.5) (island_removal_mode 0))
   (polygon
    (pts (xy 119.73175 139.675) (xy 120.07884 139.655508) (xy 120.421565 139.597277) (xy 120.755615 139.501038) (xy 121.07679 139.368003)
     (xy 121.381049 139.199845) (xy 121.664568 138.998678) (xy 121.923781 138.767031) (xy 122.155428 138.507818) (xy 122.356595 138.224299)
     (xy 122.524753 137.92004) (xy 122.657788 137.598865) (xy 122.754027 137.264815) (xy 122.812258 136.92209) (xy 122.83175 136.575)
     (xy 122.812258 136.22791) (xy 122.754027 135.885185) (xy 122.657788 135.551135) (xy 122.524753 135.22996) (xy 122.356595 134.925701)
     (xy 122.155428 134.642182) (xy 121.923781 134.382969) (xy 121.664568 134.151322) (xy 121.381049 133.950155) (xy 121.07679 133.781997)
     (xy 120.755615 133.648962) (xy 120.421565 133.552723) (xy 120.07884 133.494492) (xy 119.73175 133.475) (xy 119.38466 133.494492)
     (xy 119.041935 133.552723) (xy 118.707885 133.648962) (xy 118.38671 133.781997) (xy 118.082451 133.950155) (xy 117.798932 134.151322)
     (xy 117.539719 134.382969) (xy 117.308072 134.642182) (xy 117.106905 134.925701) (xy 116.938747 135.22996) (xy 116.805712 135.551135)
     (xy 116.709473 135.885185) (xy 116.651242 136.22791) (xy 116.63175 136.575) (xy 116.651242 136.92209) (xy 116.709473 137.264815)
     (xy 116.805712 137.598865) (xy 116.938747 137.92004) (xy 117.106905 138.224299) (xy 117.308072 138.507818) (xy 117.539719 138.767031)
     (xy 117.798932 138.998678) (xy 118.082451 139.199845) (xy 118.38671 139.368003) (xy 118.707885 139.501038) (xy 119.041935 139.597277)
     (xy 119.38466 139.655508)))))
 (gr_rect (start 62.5 72) (end 162.5 172) (stroke (width 0.05) (type solid)) (fill no) (layer "Edge.Cuts"))
 (segment (start 30 94) (end 30 92.25) (width 1) (layer "B.Cu") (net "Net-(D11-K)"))
 (segment (start 68.3675 78.35) (end 83.33 78.35) (width 1.2) (layer "B.Cu") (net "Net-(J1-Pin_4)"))
 (segment (start 83.33 78.35) (end 84.9 79.92) (width 1.2) (layer "B.Cu") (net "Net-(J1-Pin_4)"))
 (segment (start 84.84 82.52) (end 84.9 82.46) (width 1) (layer "B.Cu") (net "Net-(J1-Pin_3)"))
 (segment (start 69.2175 82.5) (end 84.86 82.5) (width 1.2) (layer "B.Cu") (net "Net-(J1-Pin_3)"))
 (segment (start 68.3675 83.35) (end 69.2175 82.5) (width 1.2) (layer "B.Cu") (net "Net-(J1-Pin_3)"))
 (segment (start 84.86 82.5) (end 84.9 82.46) (width 1.2) (layer "B.Cu") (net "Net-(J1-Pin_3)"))
 (segment (start 68.3675 88.35) (end 73.65 88.35) (width 1.2) (layer "B.Cu") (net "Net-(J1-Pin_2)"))
 (segment (start 77 85) (end 84.9 85) (width 1.2) (layer "B.Cu") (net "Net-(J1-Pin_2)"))
 (segment (start 84.84 85.06) (end 84.9 85) (width 1) (layer "B.Cu") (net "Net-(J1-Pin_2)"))
 (segment (start 73.65 88.35) (end 77 85) (width 1.2) (layer "B.Cu") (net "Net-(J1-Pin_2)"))
 (segment (start 84.9 87.54) (end 79.96 87.54) (width 1) (layer "B.Cu") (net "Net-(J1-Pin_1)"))
 (segment (start 74.15 93.35) (end 68.3675 93.35) (width 1) (layer "B.Cu") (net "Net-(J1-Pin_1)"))
 (segment (start 79.96 87.54) (end 74.15 93.35) (width 1) (layer "B.Cu") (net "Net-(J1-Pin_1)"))
 (segment (start 84.84 87.6) (end 84.9 87.54) (width 1) (layer "B.Cu") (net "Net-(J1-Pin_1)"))
 (segment (start 132.49675 87.18) (end 141.46175 96.145) (width 1.2) (layer "B.Cu") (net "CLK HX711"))
 (segment (start 109.9 87.18) (end 132.49675 87.18) (width 1.2) (layer "B.Cu") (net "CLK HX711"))
 (segment (start 132.49675 84.64) (end 141.46175 93.605) (width 1.2) (layer "B.Cu") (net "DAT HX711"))
 (segment (start 109.9 84.64) (end 132.49675 84.64) (width 1.2) (layer "B.Cu") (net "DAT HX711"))
 (segment (start 31.815 100.815) (end 31.65 100.65) (width 1) (layer "B.Cu") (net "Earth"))
 (segment (start 154.5 146) (end 156 144.5) (width 1.2) (layer "B.Cu") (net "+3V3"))
 (segment (start 156 141.5) (end 154 139.5) (width 1.2) (layer "B.Cu") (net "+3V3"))
 (segment (start 145.5 139.5) (end 141.46175 135.46175) (width 1.2) (layer "B.Cu") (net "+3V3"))
 (segment (start 130.745 144.325) (end 132.42 146) (width 1.2) (layer "B.Cu") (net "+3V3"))
 (segment (start 154 139.5) (end 145.5 139.5) (width 1.2) (layer "B.Cu") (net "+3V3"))
 (segment (start 156 144.5) (end 156 141.5) (width 1.2) (layer "B.Cu") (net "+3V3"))
 (segment (start 141.46175 135.46175) (end 141.46175 131.705) (width 1.2) (layer "B.Cu") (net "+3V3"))
 (segment (start 132.42 146) (end 154.5 146) (width 1.2) (layer "B.Cu") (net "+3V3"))
 (segment (start 130.745 143.5) (end 130.745 144.325) (width 1.2) (layer "B.Cu") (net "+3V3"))
 (segment (start 138.365 143.5) (end 138.365 130.635) (width 1.2) (layer "B.Cu") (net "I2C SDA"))
 (segment (start 139.835 129.165) (end 141.46175 129.165) (width 1.2) (layer "B.Cu") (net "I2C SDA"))
 (segment (start 138.365 130.635) (end 139.835 129.165) (width 1.2) (layer "B.Cu") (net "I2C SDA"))
 (segment (start 135.5 130) (end 135.5 143.175) (width 1.2) (layer "B.Cu") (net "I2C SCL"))
 (segment (start 138.875 126.625) (end 135.5 130) (width 1.2) (layer "B.Cu") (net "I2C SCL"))
 (segment (start 135.5 143.175) (end 135.825 143.5) (width 1.2) (layer "B.Cu") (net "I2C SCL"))
 (segment (start 141.46175 126.625) (end 138.875 126.625) (width 1.2) (layer "B.Cu") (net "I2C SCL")))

